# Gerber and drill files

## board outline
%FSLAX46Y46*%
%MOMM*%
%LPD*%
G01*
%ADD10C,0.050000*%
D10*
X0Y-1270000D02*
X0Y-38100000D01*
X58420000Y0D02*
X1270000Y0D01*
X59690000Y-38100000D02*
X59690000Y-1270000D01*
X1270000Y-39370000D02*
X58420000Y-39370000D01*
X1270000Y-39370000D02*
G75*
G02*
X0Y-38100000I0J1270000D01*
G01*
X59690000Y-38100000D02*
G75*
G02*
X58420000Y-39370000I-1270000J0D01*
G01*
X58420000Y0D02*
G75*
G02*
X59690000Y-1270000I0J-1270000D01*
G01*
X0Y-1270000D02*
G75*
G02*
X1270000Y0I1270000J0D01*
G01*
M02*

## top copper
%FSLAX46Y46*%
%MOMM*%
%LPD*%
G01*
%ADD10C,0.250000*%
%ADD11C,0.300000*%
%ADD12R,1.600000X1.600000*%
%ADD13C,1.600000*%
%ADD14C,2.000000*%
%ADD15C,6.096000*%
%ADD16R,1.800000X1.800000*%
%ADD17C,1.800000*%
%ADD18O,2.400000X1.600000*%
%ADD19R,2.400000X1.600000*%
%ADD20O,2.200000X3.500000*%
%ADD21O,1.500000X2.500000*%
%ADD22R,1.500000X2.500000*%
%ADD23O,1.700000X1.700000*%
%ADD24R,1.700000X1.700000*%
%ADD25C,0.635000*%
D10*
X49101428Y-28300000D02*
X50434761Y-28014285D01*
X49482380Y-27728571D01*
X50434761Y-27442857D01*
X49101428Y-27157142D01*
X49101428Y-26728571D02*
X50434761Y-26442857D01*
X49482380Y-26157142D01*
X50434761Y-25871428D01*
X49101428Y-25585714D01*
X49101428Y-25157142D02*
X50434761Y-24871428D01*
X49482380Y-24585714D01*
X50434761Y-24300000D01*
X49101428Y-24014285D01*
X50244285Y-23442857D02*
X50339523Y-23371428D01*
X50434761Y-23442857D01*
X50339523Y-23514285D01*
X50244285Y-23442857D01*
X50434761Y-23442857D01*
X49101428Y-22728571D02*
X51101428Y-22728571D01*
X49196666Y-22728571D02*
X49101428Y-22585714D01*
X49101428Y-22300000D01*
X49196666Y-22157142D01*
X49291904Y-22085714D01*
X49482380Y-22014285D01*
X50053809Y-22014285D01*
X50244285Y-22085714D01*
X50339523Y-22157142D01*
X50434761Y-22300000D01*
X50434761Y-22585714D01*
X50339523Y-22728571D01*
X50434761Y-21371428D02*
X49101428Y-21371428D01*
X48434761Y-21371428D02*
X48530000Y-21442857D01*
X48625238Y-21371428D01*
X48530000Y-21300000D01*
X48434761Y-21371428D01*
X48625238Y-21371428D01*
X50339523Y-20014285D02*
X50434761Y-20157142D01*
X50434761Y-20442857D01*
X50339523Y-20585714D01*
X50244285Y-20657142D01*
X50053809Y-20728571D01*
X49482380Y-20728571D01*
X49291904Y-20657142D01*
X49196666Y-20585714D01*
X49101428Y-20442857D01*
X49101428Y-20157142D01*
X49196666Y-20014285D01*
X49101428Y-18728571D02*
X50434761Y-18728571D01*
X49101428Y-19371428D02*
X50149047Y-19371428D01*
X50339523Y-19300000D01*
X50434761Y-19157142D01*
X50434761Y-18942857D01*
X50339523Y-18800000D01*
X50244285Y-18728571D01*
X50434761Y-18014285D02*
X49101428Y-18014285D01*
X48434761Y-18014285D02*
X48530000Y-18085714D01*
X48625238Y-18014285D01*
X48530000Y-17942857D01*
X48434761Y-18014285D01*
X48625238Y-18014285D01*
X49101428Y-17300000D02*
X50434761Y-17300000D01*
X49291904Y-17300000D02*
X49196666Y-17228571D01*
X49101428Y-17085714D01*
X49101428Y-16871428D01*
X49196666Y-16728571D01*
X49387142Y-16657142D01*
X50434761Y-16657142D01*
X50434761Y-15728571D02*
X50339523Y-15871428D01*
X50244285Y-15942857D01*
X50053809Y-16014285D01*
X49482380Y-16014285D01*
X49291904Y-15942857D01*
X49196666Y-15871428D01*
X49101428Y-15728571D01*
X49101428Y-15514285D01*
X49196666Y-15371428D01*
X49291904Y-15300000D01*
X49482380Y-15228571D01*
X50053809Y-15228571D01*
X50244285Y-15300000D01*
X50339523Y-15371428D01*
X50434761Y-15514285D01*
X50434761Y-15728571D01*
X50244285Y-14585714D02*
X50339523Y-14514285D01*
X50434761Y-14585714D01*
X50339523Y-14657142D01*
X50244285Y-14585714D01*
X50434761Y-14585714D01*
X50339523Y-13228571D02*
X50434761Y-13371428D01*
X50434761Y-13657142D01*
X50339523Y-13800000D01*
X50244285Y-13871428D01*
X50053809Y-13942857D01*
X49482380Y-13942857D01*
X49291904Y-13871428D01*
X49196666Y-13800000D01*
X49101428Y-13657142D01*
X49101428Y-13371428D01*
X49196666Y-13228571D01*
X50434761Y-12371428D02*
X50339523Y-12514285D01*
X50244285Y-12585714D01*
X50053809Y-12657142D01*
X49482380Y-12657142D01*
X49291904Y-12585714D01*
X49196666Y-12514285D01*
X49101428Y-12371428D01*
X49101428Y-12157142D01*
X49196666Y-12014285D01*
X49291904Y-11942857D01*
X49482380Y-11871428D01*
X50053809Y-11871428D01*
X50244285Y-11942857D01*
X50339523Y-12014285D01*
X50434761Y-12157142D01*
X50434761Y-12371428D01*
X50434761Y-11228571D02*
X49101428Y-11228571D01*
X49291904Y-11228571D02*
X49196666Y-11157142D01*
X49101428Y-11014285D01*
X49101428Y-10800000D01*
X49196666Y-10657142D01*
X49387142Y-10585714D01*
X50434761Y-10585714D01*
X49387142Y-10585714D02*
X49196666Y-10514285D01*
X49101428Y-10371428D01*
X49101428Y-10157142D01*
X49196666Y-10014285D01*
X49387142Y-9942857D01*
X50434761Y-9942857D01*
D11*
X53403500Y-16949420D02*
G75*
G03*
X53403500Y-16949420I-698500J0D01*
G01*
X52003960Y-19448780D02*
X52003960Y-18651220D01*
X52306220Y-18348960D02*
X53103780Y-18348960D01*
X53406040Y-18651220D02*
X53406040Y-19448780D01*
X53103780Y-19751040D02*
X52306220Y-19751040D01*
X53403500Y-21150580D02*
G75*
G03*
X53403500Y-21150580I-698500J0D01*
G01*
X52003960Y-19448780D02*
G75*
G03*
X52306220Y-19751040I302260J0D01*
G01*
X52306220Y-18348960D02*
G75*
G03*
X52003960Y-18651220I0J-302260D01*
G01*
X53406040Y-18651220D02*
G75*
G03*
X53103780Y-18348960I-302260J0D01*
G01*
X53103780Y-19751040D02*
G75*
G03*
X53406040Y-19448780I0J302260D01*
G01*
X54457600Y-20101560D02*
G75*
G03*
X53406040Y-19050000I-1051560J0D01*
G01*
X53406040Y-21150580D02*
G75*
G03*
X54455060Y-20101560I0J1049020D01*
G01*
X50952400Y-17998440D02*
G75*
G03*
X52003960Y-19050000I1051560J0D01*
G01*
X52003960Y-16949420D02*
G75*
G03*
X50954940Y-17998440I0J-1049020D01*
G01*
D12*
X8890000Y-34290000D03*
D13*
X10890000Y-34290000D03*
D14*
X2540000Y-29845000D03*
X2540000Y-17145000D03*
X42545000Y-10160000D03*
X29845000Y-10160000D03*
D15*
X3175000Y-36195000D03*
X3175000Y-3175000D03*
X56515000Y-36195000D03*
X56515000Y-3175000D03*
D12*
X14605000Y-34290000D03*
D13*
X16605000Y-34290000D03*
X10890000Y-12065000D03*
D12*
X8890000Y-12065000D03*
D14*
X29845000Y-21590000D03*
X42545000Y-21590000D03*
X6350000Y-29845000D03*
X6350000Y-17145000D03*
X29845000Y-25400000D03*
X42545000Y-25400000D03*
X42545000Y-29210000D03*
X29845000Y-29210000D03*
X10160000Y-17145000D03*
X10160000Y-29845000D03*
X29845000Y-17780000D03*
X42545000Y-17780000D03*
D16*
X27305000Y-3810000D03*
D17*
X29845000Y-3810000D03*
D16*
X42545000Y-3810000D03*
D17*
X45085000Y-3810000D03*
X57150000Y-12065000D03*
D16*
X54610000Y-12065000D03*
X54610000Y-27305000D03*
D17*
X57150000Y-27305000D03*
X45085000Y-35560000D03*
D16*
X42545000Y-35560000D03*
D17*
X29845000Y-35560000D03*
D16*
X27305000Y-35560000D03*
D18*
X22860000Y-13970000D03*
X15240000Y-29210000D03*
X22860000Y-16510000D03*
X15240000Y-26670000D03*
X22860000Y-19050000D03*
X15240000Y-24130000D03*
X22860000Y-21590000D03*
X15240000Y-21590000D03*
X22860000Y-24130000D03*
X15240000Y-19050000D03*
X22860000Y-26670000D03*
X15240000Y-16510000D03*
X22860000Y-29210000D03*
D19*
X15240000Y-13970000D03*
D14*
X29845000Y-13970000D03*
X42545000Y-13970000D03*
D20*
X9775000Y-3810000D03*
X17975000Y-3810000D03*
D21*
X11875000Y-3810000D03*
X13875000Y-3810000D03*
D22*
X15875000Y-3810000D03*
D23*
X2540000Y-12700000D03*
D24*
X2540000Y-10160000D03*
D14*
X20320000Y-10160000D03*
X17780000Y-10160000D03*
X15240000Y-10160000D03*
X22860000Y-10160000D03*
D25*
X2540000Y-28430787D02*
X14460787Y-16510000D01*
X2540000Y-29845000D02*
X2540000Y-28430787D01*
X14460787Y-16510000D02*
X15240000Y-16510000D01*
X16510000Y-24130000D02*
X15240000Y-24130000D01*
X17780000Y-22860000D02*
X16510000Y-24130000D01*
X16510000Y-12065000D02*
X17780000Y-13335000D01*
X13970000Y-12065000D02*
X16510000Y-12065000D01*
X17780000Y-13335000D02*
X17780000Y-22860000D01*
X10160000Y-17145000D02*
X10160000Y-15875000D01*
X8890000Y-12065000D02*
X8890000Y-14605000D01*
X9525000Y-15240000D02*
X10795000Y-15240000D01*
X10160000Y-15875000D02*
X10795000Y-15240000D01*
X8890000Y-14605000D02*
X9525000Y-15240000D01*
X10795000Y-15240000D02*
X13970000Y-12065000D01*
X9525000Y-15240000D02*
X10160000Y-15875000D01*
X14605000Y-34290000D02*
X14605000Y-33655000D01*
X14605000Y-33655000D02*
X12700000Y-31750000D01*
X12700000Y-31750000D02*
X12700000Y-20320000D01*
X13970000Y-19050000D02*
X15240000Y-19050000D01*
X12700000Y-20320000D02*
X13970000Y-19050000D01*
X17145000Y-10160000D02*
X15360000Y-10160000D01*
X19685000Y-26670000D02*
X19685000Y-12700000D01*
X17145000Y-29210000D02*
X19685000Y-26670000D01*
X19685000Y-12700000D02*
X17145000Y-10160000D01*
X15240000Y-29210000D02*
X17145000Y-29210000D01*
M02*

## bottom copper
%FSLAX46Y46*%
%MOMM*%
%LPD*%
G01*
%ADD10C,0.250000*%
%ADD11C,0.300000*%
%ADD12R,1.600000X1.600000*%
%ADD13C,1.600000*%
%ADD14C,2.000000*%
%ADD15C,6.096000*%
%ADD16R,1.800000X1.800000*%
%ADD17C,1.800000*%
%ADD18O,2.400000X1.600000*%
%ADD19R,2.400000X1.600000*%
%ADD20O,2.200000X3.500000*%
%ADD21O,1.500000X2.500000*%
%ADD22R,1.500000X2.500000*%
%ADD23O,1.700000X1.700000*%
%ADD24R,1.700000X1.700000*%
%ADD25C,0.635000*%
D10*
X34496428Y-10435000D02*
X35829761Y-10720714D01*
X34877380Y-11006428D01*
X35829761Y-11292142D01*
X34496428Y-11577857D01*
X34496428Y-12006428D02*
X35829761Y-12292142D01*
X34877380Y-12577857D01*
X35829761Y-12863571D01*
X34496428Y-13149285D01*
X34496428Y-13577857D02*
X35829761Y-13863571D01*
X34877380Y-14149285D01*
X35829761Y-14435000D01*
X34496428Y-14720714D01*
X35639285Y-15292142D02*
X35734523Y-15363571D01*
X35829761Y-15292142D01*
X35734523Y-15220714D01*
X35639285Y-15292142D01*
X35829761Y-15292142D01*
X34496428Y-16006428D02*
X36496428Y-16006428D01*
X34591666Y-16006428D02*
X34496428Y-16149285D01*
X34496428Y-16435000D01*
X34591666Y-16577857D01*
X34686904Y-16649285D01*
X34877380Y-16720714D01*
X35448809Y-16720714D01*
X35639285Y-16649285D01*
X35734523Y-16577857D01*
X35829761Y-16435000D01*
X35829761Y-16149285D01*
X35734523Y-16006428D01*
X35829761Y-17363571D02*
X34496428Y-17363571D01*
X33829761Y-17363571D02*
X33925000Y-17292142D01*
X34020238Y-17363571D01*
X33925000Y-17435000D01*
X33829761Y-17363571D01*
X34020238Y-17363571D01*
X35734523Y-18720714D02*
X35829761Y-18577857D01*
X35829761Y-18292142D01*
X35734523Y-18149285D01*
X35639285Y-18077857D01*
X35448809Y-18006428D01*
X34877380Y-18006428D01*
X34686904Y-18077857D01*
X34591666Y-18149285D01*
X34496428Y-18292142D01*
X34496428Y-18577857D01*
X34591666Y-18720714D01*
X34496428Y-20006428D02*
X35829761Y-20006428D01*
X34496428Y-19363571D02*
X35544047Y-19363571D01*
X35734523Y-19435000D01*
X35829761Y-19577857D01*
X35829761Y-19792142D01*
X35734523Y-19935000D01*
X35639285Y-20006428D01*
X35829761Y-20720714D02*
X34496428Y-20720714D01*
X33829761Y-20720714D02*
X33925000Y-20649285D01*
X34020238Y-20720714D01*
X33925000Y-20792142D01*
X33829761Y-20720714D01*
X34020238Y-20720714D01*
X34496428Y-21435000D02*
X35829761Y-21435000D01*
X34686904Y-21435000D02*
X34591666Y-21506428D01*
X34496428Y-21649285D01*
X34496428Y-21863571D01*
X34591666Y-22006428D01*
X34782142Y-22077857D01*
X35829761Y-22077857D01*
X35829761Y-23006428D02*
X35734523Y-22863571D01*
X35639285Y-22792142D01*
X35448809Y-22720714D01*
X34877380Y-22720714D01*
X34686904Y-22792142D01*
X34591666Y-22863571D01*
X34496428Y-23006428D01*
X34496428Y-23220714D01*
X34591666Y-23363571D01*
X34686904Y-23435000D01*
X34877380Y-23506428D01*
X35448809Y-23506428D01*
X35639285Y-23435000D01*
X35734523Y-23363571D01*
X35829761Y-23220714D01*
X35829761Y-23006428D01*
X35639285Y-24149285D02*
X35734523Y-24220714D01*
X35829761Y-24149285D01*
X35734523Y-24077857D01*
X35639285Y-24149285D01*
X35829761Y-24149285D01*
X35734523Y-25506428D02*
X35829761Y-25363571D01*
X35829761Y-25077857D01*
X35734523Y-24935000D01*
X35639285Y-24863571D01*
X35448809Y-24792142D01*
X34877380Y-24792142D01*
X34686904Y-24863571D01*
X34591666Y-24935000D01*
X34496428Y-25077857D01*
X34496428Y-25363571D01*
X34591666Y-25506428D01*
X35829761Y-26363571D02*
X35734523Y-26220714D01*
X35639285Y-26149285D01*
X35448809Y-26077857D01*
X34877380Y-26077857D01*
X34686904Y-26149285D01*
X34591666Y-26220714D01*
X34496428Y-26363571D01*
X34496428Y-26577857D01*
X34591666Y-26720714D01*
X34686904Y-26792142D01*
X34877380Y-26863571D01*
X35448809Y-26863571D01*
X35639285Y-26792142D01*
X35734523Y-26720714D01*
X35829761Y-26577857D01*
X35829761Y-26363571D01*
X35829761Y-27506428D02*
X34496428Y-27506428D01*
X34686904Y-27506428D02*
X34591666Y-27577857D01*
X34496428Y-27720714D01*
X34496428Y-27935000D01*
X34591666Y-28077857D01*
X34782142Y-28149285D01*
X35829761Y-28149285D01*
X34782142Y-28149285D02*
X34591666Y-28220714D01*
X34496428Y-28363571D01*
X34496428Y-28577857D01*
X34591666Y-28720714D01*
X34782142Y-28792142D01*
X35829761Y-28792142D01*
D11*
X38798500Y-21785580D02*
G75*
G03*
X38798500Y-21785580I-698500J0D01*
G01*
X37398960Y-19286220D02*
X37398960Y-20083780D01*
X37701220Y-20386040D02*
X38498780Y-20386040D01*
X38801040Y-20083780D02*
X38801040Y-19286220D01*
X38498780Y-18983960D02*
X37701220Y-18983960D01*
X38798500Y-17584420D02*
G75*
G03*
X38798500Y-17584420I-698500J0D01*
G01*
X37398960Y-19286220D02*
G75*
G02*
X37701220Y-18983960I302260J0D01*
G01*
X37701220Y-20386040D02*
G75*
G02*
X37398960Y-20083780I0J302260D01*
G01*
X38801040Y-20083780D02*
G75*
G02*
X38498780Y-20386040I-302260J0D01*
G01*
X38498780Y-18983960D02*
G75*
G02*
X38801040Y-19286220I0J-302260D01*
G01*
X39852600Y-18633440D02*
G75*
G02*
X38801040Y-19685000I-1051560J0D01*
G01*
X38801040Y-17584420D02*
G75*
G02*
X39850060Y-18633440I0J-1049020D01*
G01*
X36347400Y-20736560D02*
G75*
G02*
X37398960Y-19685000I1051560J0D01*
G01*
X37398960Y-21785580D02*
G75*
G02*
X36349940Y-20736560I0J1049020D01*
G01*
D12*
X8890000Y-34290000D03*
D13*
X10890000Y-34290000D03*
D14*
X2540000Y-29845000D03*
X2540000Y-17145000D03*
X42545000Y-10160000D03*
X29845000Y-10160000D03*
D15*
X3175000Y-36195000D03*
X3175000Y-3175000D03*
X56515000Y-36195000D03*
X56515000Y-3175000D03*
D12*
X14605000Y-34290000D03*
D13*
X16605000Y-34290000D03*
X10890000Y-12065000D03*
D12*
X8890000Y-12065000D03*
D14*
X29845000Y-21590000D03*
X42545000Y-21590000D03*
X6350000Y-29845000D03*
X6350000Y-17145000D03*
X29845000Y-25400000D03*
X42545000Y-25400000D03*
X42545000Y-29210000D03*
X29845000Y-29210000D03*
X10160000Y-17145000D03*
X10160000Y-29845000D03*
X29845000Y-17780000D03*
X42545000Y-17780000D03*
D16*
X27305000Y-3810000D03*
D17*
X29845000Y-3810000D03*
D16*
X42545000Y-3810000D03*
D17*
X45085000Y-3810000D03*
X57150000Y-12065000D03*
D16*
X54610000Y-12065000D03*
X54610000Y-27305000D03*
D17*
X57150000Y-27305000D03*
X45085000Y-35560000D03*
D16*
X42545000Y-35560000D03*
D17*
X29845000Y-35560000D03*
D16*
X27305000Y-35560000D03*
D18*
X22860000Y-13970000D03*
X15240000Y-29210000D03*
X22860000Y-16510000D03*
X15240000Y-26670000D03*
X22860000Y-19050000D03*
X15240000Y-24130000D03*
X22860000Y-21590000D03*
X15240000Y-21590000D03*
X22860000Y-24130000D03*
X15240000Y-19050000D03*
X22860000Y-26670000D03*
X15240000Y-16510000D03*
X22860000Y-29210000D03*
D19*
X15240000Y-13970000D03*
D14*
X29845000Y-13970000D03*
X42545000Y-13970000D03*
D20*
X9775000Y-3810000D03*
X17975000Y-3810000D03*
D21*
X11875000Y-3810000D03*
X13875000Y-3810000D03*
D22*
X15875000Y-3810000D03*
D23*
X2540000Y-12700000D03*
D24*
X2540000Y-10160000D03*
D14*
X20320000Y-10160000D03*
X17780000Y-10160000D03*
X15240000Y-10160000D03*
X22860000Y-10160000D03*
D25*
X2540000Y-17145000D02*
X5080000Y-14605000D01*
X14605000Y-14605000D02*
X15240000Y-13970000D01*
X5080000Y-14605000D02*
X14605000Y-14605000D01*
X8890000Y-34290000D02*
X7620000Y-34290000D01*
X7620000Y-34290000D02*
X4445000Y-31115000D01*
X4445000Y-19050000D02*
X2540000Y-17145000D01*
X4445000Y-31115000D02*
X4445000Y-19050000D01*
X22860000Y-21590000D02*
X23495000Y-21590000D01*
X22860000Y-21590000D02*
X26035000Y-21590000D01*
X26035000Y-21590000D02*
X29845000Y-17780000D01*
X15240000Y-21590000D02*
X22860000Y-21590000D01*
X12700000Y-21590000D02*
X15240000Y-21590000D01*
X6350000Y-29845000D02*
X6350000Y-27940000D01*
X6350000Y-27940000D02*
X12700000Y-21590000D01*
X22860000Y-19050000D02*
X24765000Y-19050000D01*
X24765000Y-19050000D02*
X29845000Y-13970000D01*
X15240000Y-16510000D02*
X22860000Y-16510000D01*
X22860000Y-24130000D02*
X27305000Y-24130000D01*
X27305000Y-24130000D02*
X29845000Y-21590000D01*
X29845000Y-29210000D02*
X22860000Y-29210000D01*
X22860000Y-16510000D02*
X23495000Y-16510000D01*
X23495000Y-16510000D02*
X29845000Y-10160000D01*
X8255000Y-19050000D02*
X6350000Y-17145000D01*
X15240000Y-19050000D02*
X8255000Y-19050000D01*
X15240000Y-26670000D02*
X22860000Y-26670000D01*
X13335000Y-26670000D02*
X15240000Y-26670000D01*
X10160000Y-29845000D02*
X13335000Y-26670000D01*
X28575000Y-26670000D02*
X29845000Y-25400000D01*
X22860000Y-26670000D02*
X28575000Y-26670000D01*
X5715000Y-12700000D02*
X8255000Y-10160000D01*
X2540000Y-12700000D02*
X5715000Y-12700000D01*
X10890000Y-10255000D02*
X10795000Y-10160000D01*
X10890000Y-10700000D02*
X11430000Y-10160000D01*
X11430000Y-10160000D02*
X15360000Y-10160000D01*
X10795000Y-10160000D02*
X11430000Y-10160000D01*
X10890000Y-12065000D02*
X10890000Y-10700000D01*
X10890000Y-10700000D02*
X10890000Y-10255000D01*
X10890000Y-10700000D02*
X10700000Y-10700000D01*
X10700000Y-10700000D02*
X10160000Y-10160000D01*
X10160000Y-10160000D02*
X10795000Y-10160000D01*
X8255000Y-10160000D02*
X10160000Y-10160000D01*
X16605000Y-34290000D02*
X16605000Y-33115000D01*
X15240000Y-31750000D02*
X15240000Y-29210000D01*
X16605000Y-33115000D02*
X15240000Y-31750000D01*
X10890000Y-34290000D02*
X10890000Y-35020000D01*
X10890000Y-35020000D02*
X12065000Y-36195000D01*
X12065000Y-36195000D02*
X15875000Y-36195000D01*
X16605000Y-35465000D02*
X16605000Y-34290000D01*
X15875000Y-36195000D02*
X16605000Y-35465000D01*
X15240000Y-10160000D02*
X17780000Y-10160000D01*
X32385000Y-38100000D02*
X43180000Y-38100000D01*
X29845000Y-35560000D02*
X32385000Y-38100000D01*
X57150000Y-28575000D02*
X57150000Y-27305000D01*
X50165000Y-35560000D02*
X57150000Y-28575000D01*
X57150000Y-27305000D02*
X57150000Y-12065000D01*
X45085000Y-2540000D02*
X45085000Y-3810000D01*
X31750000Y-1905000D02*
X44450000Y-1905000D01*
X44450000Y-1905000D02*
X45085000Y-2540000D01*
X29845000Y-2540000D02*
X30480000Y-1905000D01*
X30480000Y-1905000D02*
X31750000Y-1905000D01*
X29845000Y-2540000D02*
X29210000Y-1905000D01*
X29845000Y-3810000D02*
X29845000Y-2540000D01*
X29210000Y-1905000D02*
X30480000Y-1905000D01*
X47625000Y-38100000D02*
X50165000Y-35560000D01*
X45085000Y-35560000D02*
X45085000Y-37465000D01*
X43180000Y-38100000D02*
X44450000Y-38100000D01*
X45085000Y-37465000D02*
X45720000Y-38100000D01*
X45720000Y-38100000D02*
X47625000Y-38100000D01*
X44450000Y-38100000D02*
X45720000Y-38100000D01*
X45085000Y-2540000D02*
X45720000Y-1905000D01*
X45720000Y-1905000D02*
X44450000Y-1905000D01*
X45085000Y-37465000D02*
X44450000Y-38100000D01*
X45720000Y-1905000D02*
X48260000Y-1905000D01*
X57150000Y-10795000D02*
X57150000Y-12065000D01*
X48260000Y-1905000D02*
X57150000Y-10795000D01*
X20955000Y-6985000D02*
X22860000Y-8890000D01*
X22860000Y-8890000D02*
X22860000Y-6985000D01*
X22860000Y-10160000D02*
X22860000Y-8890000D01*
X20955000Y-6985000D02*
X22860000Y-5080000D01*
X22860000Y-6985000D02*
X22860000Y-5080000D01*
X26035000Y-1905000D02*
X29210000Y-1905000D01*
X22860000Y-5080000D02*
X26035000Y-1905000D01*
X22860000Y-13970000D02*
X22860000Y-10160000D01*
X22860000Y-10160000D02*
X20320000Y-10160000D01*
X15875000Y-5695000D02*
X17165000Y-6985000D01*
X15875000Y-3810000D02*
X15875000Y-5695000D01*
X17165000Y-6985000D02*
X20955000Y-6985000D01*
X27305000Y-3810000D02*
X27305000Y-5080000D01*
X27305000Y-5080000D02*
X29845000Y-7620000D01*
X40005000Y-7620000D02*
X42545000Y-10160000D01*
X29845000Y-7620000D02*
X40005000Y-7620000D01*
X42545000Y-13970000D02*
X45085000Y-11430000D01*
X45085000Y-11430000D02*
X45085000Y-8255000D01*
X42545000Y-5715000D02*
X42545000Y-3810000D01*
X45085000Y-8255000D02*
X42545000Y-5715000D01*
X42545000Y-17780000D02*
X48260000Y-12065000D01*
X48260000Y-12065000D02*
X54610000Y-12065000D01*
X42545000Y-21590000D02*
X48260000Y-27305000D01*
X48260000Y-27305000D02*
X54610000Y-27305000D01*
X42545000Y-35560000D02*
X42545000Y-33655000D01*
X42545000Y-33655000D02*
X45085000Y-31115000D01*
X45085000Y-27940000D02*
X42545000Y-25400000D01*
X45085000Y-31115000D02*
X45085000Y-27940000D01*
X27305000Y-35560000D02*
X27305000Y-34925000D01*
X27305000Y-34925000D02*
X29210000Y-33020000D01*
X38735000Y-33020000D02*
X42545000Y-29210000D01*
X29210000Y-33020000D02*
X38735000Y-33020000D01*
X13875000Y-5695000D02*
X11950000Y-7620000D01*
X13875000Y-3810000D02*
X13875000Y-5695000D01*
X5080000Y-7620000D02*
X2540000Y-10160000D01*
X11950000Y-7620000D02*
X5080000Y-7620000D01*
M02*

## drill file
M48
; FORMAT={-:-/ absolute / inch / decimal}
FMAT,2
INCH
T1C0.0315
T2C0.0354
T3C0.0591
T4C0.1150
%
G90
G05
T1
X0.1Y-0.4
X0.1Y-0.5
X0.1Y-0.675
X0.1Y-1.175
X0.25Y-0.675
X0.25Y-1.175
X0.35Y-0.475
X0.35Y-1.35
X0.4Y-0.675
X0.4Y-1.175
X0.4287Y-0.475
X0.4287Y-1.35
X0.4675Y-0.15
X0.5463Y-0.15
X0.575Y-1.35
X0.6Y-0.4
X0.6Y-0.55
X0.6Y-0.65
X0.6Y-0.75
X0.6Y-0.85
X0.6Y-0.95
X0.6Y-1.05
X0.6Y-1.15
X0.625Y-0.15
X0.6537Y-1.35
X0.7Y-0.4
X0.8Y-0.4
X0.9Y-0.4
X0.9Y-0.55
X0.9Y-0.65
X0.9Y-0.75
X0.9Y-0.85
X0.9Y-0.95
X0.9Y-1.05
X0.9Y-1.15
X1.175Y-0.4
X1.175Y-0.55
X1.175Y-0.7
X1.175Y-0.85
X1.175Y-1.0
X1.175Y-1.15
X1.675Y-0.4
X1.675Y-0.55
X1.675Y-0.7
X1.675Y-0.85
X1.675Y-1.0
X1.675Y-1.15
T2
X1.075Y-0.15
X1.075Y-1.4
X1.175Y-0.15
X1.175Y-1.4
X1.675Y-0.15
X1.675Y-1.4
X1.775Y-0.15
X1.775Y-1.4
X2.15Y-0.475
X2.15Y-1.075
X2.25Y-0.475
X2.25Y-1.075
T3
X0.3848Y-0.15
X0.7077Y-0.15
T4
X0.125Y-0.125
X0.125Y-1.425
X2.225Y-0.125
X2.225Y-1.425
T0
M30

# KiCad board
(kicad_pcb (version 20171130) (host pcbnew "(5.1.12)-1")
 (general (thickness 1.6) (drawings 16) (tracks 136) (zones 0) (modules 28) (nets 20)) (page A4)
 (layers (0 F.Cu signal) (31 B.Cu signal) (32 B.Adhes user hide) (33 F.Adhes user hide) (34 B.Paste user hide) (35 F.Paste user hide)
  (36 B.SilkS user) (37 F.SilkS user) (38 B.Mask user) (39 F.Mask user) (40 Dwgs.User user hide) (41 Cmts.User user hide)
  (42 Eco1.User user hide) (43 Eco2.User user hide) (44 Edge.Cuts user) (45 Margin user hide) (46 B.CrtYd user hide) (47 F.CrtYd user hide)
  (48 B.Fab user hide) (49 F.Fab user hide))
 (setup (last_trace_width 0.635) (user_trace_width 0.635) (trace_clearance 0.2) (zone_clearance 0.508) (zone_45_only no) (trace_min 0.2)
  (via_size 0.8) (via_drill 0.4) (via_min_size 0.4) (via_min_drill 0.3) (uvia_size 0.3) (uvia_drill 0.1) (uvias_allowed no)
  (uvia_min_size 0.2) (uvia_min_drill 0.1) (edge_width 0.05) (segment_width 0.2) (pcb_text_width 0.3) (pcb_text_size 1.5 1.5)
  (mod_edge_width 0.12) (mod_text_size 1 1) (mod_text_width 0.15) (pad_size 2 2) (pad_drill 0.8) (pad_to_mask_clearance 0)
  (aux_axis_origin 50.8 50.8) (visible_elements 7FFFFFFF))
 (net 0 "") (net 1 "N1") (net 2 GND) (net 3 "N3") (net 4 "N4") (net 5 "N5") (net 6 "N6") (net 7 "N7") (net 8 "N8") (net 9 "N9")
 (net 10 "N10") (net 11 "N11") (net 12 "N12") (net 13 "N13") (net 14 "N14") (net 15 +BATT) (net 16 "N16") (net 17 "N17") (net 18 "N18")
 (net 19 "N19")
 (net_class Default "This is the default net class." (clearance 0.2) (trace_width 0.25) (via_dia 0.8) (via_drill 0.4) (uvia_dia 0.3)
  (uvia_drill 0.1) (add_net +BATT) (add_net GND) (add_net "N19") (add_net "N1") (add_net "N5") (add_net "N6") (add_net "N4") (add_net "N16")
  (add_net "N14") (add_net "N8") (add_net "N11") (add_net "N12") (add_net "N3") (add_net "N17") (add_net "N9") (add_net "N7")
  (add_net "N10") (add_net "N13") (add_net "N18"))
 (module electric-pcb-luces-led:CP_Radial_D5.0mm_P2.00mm (layer F.Cu) (at 59.69 85.09)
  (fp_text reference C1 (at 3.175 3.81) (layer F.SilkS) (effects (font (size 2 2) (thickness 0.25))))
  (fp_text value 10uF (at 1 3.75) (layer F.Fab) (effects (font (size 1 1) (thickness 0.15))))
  (pad 1 thru_hole rect (at 0 0) (size 1.6 1.6) (drill 0.8) (layers *.Cu *.Mask) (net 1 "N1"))
  (pad 2 thru_hole circle (at 2 0) (size 1.6 1.6) (drill 0.8) (layers *.Cu *.Mask) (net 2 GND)))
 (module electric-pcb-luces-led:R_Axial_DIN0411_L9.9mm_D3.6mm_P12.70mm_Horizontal (layer F.Cu) (at 53.34 80.645 90)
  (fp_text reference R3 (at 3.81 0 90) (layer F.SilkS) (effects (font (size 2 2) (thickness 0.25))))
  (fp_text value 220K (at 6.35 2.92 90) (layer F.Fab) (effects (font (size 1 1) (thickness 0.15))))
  (pad 1 thru_hole circle (at 0 0 90) (size 2 2) (drill 0.8) (layers *.Cu *.Mask) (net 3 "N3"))
  (pad 2 thru_hole circle (at 12.7 0 90) (size 2 2) (drill 0.8) (layers *.Cu *.Mask) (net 1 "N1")))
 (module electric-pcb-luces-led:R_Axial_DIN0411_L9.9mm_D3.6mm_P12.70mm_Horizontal (layer F.Cu) (at 93.345 60.96 180)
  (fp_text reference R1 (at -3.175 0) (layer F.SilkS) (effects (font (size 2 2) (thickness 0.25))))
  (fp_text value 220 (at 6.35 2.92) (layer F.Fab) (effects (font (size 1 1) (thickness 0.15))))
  (pad 1 thru_hole circle (at 0 0 180) (size 2 2) (drill 0.8) (layers *.Cu *.Mask) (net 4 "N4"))
  (pad 2 thru_hole circle (at 12.7 0 180) (size 2 2) (drill 0.8) (layers *.Cu *.Mask) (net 3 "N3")))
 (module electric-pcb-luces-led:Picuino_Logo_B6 (layer B.Cu) (at 103.505 69.85 270)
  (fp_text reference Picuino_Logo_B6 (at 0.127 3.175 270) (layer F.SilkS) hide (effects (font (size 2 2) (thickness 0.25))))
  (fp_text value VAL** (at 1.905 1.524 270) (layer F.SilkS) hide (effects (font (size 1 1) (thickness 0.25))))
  (fp_circle (center -2.10058 0) (end -1.40208 0) (layer F.Cu) (width 0.3))
  (fp_line (start 0.39878 0.70104) (end -0.39878 0.70104) (layer F.Cu) (width 0.3))
  (fp_line (start -0.70104 0.39878) (end -0.70104 -0.39878) (layer F.Cu) (width 0.3))
  (fp_line (start -0.39878 -0.70104) (end 0.39878 -0.70104) (layer F.Cu) (width 0.3))
  (fp_line (start 0.70104 -0.39878) (end 0.70104 0.39878) (layer F.Cu) (width 0.3))
  (fp_circle (center 2.10058 0) (end 2.79908 0) (layer F.Cu) (width 0.3))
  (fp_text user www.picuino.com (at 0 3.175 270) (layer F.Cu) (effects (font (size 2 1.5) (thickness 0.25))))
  (fp_arc (start 0.39878 0.39878) (end 0.70104 0.39878) (angle 90) (layer F.Cu) (width 0.3))
  (fp_arc (start -0.39878 0.39878) (end -0.39878 0.70104) (angle 90) (layer F.Cu) (width 0.3))
  (fp_arc (start -0.39878 -0.39878) (end -0.70104 -0.39878) (angle 90) (layer F.Cu) (width 0.3))
  (fp_arc (start 0.39878 -0.39878) (end 0.39878 -0.70104) (angle 90) (layer F.Cu) (width 0.3))
  (fp_arc (start 1.05156 -0.70104) (end 0 -0.70104) (angle 90) (layer F.Cu) (width 0.3))
  (fp_arc (start 1.05156 -0.70104) (end 1.05156 -1.75006) (angle 90) (layer F.Cu) (width 0.3))
  (fp_arc (start -1.05156 0.70104) (end 0 0.70104) (angle 90) (layer F.Cu) (width 0.3))
  (fp_arc (start -1.05156 0.70104) (end -1.05156 1.75006) (angle 90) (layer F.Cu) (width 0.3)))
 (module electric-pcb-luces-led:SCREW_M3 (layer F.Cu) (at 53.975 86.995)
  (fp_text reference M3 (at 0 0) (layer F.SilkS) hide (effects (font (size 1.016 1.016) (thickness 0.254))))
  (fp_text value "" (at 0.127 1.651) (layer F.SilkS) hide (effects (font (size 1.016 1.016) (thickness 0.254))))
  (pad "" thru_hole circle (at 0 0) (size 6.096 6.096) (drill 2.921) (layers *.Cu F.SilkS)))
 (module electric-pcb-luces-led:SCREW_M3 (layer F.Cu) (at 53.975 53.975)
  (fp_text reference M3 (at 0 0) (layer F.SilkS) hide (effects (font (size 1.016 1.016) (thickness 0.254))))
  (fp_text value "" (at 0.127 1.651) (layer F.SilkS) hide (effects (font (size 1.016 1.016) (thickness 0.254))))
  (pad "" thru_hole circle (at 0 0) (size 6.096 6.096) (drill 2.921) (layers *.Cu F.SilkS)))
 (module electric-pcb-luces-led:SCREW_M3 (layer F.Cu) (at 107.315 86.995)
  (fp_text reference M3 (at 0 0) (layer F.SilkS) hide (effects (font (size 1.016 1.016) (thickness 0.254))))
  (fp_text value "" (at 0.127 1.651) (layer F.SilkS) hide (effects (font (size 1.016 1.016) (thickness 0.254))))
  (pad "" thru_hole circle (at 0 0) (size 6.096 6.096) (drill 2.921) (layers *.Cu F.SilkS)))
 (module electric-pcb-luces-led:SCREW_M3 (layer F.Cu) (at 107.315 53.975)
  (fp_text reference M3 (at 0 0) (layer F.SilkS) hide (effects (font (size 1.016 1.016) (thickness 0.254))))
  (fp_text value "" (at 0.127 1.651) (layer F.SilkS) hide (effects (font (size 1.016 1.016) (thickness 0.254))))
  (pad "" thru_hole circle (at 0 0) (size 6.096 6.096) (drill 2.921) (layers *.Cu F.SilkS)))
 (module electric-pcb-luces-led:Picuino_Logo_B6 (layer F.Cu) (at 88.9 70.485 90)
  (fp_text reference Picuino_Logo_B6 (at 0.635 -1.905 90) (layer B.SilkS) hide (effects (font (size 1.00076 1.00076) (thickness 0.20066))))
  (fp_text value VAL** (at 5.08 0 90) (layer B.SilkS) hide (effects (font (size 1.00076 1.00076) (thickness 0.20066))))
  (fp_circle (center -2.10058 0) (end -1.40208 0) (layer B.Cu) (width 0.3))
  (fp_line (start 0.39878 -0.70104) (end -0.39878 -0.70104) (layer B.Cu) (width 0.3))
  (fp_line (start -0.70104 -0.39878) (end -0.70104 0.39878) (layer B.Cu) (width 0.3))
  (fp_line (start -0.39878 0.70104) (end 0.39878 0.70104) (layer B.Cu) (width 0.3))
  (fp_line (start 0.70104 0.39878) (end 0.70104 -0.39878) (layer B.Cu) (width 0.3))
  (fp_circle (center 2.10058 0) (end 2.79908 0) (layer B.Cu) (width 0.3))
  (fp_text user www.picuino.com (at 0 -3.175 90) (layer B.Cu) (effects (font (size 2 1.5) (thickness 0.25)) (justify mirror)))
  (fp_arc (start 0.39878 -0.39878) (end 0.70104 -0.39878) (angle -90) (layer B.Cu) (width 0.3))
  (fp_arc (start -0.39878 -0.39878) (end -0.39878 -0.70104) (angle -90) (layer B.Cu) (width 0.3))
  (fp_arc (start -0.39878 0.39878) (end -0.70104 0.39878) (angle -90) (layer B.Cu) (width 0.3))
  (fp_arc (start 0.39878 0.39878) (end 0.39878 0.70104) (angle -90) (layer B.Cu) (width 0.3))
  (fp_arc (start 1.05156 0.70104) (end 0 0.70104) (angle -90) (layer B.Cu) (width 0.3))
  (fp_arc (start 1.05156 0.70104) (end 1.05156 1.75006) (angle -90) (layer B.Cu) (width 0.3))
  (fp_arc (start -1.05156 -0.70104) (end 0 -0.70104) (angle -90) (layer B.Cu) (width 0.3))
  (fp_arc (start -1.05156 -0.70104) (end -1.05156 -1.75006) (angle -90) (layer B.Cu) (width 0.3)))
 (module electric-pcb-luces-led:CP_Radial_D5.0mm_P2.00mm (layer F.Cu) (at 65.405 85.09)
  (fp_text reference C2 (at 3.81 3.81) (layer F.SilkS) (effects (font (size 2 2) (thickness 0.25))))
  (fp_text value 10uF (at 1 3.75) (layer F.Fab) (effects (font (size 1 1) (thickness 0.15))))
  (pad 1 thru_hole rect (at 0 0) (size 1.6 1.6) (drill 0.8) (layers *.Cu *.Mask) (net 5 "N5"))
  (pad 2 thru_hole circle (at 2 0) (size 1.6 1.6) (drill 0.8) (layers *.Cu *.Mask) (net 2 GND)))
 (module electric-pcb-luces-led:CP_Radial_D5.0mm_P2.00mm (layer F.Cu) (at 59.69 62.865)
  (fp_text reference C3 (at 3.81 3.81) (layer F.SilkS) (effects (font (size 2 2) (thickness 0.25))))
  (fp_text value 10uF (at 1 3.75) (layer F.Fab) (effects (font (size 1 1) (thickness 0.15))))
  (pad 2 thru_hole circle (at 2 0) (size 1.6 1.6) (drill 0.8) (layers *.Cu *.Mask) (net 2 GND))
  (pad 1 thru_hole rect (at 0 0) (size 1.6 1.6) (drill 0.8) (layers *.Cu *.Mask) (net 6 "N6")))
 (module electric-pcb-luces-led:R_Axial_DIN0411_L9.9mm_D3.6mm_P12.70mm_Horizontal (layer F.Cu) (at 93.345 72.39 180)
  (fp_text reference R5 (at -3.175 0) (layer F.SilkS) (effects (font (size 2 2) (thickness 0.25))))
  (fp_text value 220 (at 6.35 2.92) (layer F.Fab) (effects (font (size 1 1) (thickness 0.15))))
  (pad 2 thru_hole circle (at 12.7 0 180) (size 2 2) (drill 0.8) (layers *.Cu *.Mask) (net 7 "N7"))
  (pad 1 thru_hole circle (at 0 0 180) (size 2 2) (drill 0.8) (layers *.Cu *.Mask) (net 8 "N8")))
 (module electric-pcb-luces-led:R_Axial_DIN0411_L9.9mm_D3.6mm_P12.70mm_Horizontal (layer F.Cu) (at 57.15 80.645 90)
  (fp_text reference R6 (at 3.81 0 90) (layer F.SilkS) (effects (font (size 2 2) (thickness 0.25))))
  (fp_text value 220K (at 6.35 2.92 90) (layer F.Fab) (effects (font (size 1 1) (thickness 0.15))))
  (pad 1 thru_hole circle (at 0 0 90) (size 2 2) (drill 0.8) (layers *.Cu *.Mask) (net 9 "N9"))
  (pad 2 thru_hole circle (at 12.7 0 90) (size 2 2) (drill 0.8) (layers *.Cu *.Mask) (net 5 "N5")))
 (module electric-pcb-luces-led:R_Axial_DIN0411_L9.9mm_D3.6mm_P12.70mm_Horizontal (layer F.Cu) (at 93.345 76.2 180)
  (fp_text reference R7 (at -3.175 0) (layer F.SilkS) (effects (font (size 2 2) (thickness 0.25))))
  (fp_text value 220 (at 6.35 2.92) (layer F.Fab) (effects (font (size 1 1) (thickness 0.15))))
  (pad 2 thru_hole circle (at 12.7 0 180) (size 2 2) (drill 0.8) (layers *.Cu *.Mask) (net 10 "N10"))
  (pad 1 thru_hole circle (at 0 0 180) (size 2 2) (drill 0.8) (layers *.Cu *.Mask) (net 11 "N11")))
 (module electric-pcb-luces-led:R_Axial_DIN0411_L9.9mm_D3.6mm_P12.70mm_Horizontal (layer F.Cu) (at 93.345 80.01 180)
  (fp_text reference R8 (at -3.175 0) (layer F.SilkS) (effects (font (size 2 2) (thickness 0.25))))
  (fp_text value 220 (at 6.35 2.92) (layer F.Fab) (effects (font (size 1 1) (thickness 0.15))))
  (pad 1 thru_hole circle (at 0 0 180) (size 2 2) (drill 0.8) (layers *.Cu *.Mask) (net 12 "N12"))
  (pad 2 thru_hole circle (at 12.7 0 180) (size 2 2) (drill 0.8) (layers *.Cu *.Mask) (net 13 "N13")))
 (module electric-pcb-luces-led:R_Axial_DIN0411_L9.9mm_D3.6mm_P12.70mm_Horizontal (layer F.Cu) (at 60.96 80.645 90)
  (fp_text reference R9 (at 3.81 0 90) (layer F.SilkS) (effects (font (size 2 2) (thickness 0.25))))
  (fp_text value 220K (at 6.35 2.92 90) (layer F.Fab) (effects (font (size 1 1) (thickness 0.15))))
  (pad 2 thru_hole circle (at 12.7 0 90) (size 2 2) (drill 0.8) (layers *.Cu *.Mask) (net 6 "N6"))
  (pad 1 thru_hole circle (at 0 0 90) (size 2 2) (drill 0.8) (layers *.Cu *.Mask) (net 10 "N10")))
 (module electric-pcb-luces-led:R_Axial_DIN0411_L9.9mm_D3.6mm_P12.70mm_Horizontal (layer F.Cu) (at 93.345 68.58 180)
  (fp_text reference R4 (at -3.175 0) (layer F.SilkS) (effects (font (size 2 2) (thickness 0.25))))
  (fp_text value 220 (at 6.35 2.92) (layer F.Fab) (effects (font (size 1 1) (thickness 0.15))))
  (pad 2 thru_hole circle (at 12.7 0 180) (size 2 2) (drill 0.8) (layers *.Cu *.Mask) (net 9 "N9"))
  (pad 1 thru_hole circle (at 0 0 180) (size 2 2) (drill 0.8) (layers *.Cu *.Mask) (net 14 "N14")))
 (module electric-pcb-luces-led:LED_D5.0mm (layer F.Cu) (at 78.105 54.61)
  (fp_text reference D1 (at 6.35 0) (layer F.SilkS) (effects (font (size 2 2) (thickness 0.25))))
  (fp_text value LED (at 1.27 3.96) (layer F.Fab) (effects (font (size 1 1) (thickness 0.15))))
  (pad 1 thru_hole rect (at 0 0) (size 1.8 1.8) (drill 0.9) (layers *.Cu *.Mask) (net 4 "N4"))
  (pad 2 thru_hole circle (at 2.54 0) (size 1.8 1.8) (drill 0.9) (layers *.Cu *.Mask) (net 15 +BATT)))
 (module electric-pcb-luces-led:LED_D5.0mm (layer F.Cu) (at 93.345 54.61)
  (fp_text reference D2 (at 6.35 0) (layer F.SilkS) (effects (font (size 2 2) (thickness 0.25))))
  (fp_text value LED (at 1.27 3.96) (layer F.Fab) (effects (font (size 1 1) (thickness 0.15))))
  (pad 1 thru_hole rect (at 0 0) (size 1.8 1.8) (drill 0.9) (layers *.Cu *.Mask) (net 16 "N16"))
  (pad 2 thru_hole circle (at 2.54 0) (size 1.8 1.8) (drill 0.9) (layers *.Cu *.Mask) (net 15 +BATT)))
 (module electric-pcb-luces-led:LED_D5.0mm (layer F.Cu) (at 105.41 62.865)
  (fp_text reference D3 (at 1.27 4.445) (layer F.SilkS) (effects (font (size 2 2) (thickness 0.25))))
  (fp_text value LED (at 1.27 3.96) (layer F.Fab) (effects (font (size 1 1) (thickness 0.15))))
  (pad 2 thru_hole circle (at 2.54 0) (size 1.8 1.8) (drill 0.9) (layers *.Cu *.Mask) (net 15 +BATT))
  (pad 1 thru_hole rect (at 0 0) (size 1.8 1.8) (drill 0.9) (layers *.Cu *.Mask) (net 14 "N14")))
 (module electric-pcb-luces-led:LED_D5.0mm (layer F.Cu) (at 105.41 78.105)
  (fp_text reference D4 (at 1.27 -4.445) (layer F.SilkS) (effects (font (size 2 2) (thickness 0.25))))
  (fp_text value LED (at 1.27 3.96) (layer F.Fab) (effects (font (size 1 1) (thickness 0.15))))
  (pad 1 thru_hole rect (at 0 0) (size 1.8 1.8) (drill 0.9) (layers *.Cu *.Mask) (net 8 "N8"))
  (pad 2 thru_hole circle (at 2.54 0) (size 1.8 1.8) (drill 0.9) (layers *.Cu *.Mask) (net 15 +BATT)))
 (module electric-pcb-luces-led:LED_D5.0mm (layer F.Cu) (at 93.345 86.36)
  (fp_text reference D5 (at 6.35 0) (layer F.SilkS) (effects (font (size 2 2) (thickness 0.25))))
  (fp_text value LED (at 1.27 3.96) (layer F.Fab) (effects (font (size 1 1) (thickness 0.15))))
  (pad 2 thru_hole circle (at 2.54 0) (size 1.8 1.8) (drill 0.9) (layers *.Cu *.Mask) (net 15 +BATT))
  (pad 1 thru_hole rect (at 0 0) (size 1.8 1.8) (drill 0.9) (layers *.Cu *.Mask) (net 11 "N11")))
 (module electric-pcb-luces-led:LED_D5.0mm (layer F.Cu) (at 78.105 86.36)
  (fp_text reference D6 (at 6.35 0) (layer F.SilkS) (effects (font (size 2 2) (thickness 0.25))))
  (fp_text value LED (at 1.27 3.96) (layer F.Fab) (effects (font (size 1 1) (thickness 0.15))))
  (pad 2 thru_hole circle (at 2.54 0) (size 1.8 1.8) (drill 0.9) (layers *.Cu *.Mask) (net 15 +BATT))
  (pad 1 thru_hole rect (at 0 0) (size 1.8 1.8) (drill 0.9) (layers *.Cu *.Mask) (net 12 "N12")))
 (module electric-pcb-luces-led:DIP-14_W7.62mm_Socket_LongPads (layer F.Cu) (at 66.04 64.77)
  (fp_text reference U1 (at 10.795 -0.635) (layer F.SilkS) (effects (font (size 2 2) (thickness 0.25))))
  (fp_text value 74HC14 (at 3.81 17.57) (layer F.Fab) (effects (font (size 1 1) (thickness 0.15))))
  (pad 14 thru_hole oval (at 7.62 0) (size 2.4 1.6) (drill 0.8) (layers *.Cu *.Mask) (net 15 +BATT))
  (pad 7 thru_hole oval (at 0 15.24) (size 2.4 1.6) (drill 0.8) (layers *.Cu *.Mask) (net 2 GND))
  (pad 13 thru_hole oval (at 7.62 2.54) (size 2.4 1.6) (drill 0.8) (layers *.Cu *.Mask) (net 3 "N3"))
  (pad 6 thru_hole oval (at 0 12.7) (size 2.4 1.6) (drill 0.8) (layers *.Cu *.Mask) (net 10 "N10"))
  (pad 12 thru_hole oval (at 7.62 5.08) (size 2.4 1.6) (drill 0.8) (layers *.Cu *.Mask) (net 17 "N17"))
  (pad 5 thru_hole oval (at 0 10.16) (size 2.4 1.6) (drill 0.8) (layers *.Cu *.Mask) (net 6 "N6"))
  (pad 11 thru_hole oval (at 7.62 7.62) (size 2.4 1.6) (drill 0.8) (layers *.Cu *.Mask) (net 9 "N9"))
  (pad 4 thru_hole oval (at 0 7.62) (size 2.4 1.6) (drill 0.8) (layers *.Cu *.Mask) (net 9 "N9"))
  (pad 10 thru_hole oval (at 7.62 10.16) (size 2.4 1.6) (drill 0.8) (layers *.Cu *.Mask) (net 7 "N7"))
  (pad 3 thru_hole oval (at 0 5.08) (size 2.4 1.6) (drill 0.8) (layers *.Cu *.Mask) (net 5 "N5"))
  (pad 9 thru_hole oval (at 7.62 12.7) (size 2.4 1.6) (drill 0.8) (layers *.Cu *.Mask) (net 10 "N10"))
  (pad 2 thru_hole oval (at 0 2.54) (size 2.4 1.6) (drill 0.8) (layers *.Cu *.Mask) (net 3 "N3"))
  (pad 8 thru_hole oval (at 7.62 15.24) (size 2.4 1.6) (drill 0.8) (layers *.Cu *.Mask) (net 13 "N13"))
  (pad 1 thru_hole rect (at 0 0) (size 2.4 1.6) (drill 0.8) (layers *.Cu *.Mask) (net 1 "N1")))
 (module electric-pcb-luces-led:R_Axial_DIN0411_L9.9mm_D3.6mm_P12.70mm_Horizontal (layer F.Cu) (at 93.345 64.77 180)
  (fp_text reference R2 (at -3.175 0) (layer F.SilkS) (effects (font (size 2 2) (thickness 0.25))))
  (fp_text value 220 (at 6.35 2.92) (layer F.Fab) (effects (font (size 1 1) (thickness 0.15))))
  (pad 2 thru_hole circle (at 12.7 0 180) (size 2 2) (drill 0.8) (layers *.Cu *.Mask) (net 17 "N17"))
  (pad 1 thru_hole circle (at 0 0 180) (size 2 2) (drill 0.8) (layers *.Cu *.Mask) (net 16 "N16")))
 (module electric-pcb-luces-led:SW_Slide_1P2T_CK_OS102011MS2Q (layer F.Cu) (at 66.675 54.61 180)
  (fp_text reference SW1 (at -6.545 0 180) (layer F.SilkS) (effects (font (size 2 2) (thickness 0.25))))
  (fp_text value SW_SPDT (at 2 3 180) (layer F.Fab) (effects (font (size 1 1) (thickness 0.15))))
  (pad "" thru_hole oval (at 6.1 0 180) (size 2.2 3.5) (drill 1.5) (layers *.Cu *.Mask))
  (pad "" thru_hole oval (at -2.1 0 180) (size 2.2 3.5) (drill 1.5) (layers *.Cu *.Mask))
  (pad 3 thru_hole oval (at 4 0 180) (size 1.5 2.5) (drill 0.8) (layers *.Cu *.Mask) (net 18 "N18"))
  (pad 2 thru_hole oval (at 2 0 180) (size 1.5 2.5) (drill 0.8) (layers *.Cu *.Mask) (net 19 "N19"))
  (pad 1 thru_hole rect (at 0 0 180) (size 1.5 2.5) (drill 0.8) (layers *.Cu *.Mask) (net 15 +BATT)))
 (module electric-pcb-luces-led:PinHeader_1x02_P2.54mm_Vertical (layer F.Cu) (at 53.34 60.96)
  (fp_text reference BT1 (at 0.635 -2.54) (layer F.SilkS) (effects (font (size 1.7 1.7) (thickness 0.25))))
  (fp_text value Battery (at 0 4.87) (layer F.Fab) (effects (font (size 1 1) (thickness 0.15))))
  (pad 2 thru_hole oval (at 0 2.54) (size 1.7 1.7) (drill 0.8) (layers *.Cu *.Mask) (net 2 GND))
  (pad 1 thru_hole rect (at 0 0) (size 1.7 1.7) (drill 0.8) (layers *.Cu *.Mask) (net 19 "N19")))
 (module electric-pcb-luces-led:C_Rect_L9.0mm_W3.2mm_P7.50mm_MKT (layer F.Cu) (at 73.66 60.96 180)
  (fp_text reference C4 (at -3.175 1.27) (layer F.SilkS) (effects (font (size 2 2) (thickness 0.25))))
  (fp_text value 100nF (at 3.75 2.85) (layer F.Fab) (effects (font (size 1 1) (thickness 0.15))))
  (pad 1 thru_hole circle (at 2.54 0 180) (size 2 2) (drill 0.8) (layers *.Cu *.Mask) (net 15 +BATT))
  (pad 2 thru_hole circle (at 5.08 0 180) (size 2 2) (drill 0.8) (layers *.Cu *.Mask) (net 2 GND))
  (pad 2 thru_hole circle (at 7.62 0 180) (size 2 2) (drill 0.8) (layers *.Cu *.Mask) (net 2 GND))
  (pad 1 thru_hole circle (at 0 0 180) (size 2 2) (drill 0.8) (layers *.Cu *.Mask) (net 15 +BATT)))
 (gr_line (start 50.8 52.07) (end 50.8 88.9) (layer Edge.Cuts) (width 0.05))
 (gr_line (start 109.22 50.8) (end 52.07 50.8) (layer Edge.Cuts) (width 0.05))
 (gr_line (start 110.49 88.9) (end 110.49 52.07) (layer Edge.Cuts) (width 0.05))
 (gr_line (start 52.07 90.17) (end 109.22 90.17) (layer Edge.Cuts) (width 0.05))
 (gr_arc (start 52.07 88.9) (end 50.8 88.9) (angle -90) (layer Edge.Cuts) (width 0.05))
 (gr_arc (start 109.22 88.9) (end 109.22 90.17) (angle -90) (layer Edge.Cuts) (width 0.05))
 (gr_arc (start 109.22 52.07) (end 110.49 52.07) (angle -90) (layer Edge.Cuts) (width 0.05))
 (gr_arc (start 52.07 52.07) (end 52.07 50.8) (angle -90) (layer Edge.Cuts) (width 0.05))
 (segment (start 53.34 67.945) (end 55.88 65.405) (width 0.635) (layer B.Cu) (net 1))
 (segment (start 65.405 65.405) (end 66.04 64.77) (width 0.635) (layer B.Cu) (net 1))
 (segment (start 55.88 65.405) (end 65.405 65.405) (width 0.635) (layer B.Cu) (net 1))
 (segment (start 59.69 85.09) (end 58.42 85.09) (width 0.635) (layer B.Cu) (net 1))
 (segment (start 58.42 85.09) (end 55.245 81.915) (width 0.635) (layer B.Cu) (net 1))
 (segment (start 55.245 69.85) (end 53.34 67.945) (width 0.635) (layer B.Cu) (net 1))
 (segment (start 55.245 81.915) (end 55.245 69.85) (width 0.635) (layer B.Cu) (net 1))
 (segment (start 73.66 72.39) (end 74.295 72.39) (width 0.635) (layer B.Cu) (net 9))
 (segment (start 73.66 72.39) (end 76.835 72.39) (width 0.635) (layer B.Cu) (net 9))
 (segment (start 76.835 72.39) (end 80.645 68.58) (width 0.635) (layer B.Cu) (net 9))
 (segment (start 66.04 72.39) (end 73.66 72.39) (width 0.635) (layer B.Cu) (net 9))
 (segment (start 63.5 72.39) (end 66.04 72.39) (width 0.635) (layer B.Cu) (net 9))
 (segment (start 57.15 80.645) (end 57.15 78.74) (width 0.635) (layer B.Cu) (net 9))
 (segment (start 57.15 78.74) (end 63.5 72.39) (width 0.635) (layer B.Cu) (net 9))
 (segment (start 73.66 69.85) (end 75.565 69.85) (width 0.635) (layer B.Cu) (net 17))
 (segment (start 75.565 69.85) (end 80.645 64.77) (width 0.635) (layer B.Cu) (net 17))
 (segment (start 66.04 67.31) (end 73.66 67.31) (width 0.635) (layer B.Cu) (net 3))
 (segment (start 73.66 74.93) (end 78.105 74.93) (width 0.635) (layer B.Cu) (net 7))
 (segment (start 78.105 74.93) (end 80.645 72.39) (width 0.635) (layer B.Cu) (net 7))
 (segment (start 80.645 80.01) (end 73.66 80.01) (width 0.635) (layer B.Cu) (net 13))
 (segment (start 53.34 79.230787) (end 65.260787 67.31) (width 0.635) (layer F.Cu) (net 3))
 (segment (start 53.34 80.645) (end 53.34 79.230787) (width 0.635) (layer F.Cu) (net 3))
 (segment (start 65.260787 67.31) (end 66.04 67.31) (width 0.635) (layer F.Cu) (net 3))
 (segment (start 73.66 67.31) (end 74.295 67.31) (width 0.635) (layer B.Cu) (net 3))
 (segment (start 74.295 67.31) (end 80.645 60.96) (width 0.635) (layer B.Cu) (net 3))
 (segment (start 67.31 74.93) (end 66.04 74.93) (width 0.635) (layer F.Cu) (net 6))
 (segment (start 68.58 73.66) (end 67.31 74.93) (width 0.635) (layer F.Cu) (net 6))
 (segment (start 67.31 62.865) (end 68.58 64.135) (width 0.635) (layer F.Cu) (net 6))
 (segment (start 64.77 62.865) (end 67.31 62.865) (width 0.635) (layer F.Cu) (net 6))
 (segment (start 68.58 64.135) (end 68.58 73.66) (width 0.635) (layer F.Cu) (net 6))
 (segment (start 60.96 67.945) (end 60.96 66.675) (width 0.635) (layer F.Cu) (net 6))
 (segment (start 59.69 62.865) (end 59.69 65.405) (width 0.635) (layer F.Cu) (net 6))
 (segment (start 60.325 66.04) (end 61.595 66.04) (width 0.635) (layer F.Cu) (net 6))
 (segment (start 60.96 66.675) (end 61.595 66.04) (width 0.635) (layer F.Cu) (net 6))
 (segment (start 59.69 65.405) (end 60.325 66.04) (width 0.635) (layer F.Cu) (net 6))
 (segment (start 61.595 66.04) (end 64.77 62.865) (width 0.635) (layer F.Cu) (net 6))
 (segment (start 60.325 66.04) (end 60.96 66.675) (width 0.635) (layer F.Cu) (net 6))
 (segment (start 59.055 69.85) (end 57.15 67.945) (width 0.635) (layer B.Cu) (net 5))
 (segment (start 66.04 69.85) (end 59.055 69.85) (width 0.635) (layer B.Cu) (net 5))
 (segment (start 65.405 85.09) (end 65.405 84.455) (width 0.635) (layer F.Cu) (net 5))
 (segment (start 65.405 84.455) (end 63.5 82.55) (width 0.635) (layer F.Cu) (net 5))
 (segment (start 63.5 82.55) (end 63.5 71.12) (width 0.635) (layer F.Cu) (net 5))
 (segment (start 64.77 69.85) (end 66.04 69.85) (width 0.635) (layer F.Cu) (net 5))
 (segment (start 63.5 71.12) (end 64.77 69.85) (width 0.635) (layer F.Cu) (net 5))
 (segment (start 66.04 77.47) (end 73.66 77.47) (width 0.635) (layer B.Cu) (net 10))
 (segment (start 64.135 77.47) (end 66.04 77.47) (width 0.635) (layer B.Cu) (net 10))
 (segment (start 60.96 80.645) (end 64.135 77.47) (width 0.635) (layer B.Cu) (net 10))
 (segment (start 79.375 77.47) (end 80.645 76.2) (width 0.635) (layer B.Cu) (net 10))
 (segment (start 73.66 77.47) (end 79.375 77.47) (width 0.635) (layer B.Cu) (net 10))
 (segment (start 67.945 60.96) (end 66.16 60.96) (width 0.635) (layer F.Cu) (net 2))
 (segment (start 70.485 77.47) (end 70.485 63.5) (width 0.635) (layer F.Cu) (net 2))
 (segment (start 67.945 80.01) (end 70.485 77.47) (width 0.635) (layer F.Cu) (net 2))
 (segment (start 70.485 63.5) (end 67.945 60.96) (width 0.635) (layer F.Cu) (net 2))
 (segment (start 66.04 80.01) (end 67.945 80.01) (width 0.635) (layer F.Cu) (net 2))
 (segment (start 56.515 63.5) (end 59.055 60.96) (width 0.635) (layer B.Cu) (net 2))
 (segment (start 53.34 63.5) (end 56.515 63.5) (width 0.635) (layer B.Cu) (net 2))
 (segment (start 61.69 61.055) (end 61.595 60.96) (width 0.635) (layer B.Cu) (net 2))
 (segment (start 61.69 61.5) (end 62.23 60.96) (width 0.635) (layer B.Cu) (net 2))
 (segment (start 62.23 60.96) (end 66.16 60.96) (width 0.635) (layer B.Cu) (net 2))
 (segment (start 61.595 60.96) (end 62.23 60.96) (width 0.635) (layer B.Cu) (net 2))
 (segment (start 61.69 62.865) (end 61.69 61.5) (width 0.635) (layer B.Cu) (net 2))
 (segment (start 61.69 61.5) (end 61.69 61.055) (width 0.635) (layer B.Cu) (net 2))
 (segment (start 61.69 61.5) (end 61.5 61.5) (width 0.635) (layer B.Cu) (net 2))
 (segment (start 61.5 61.5) (end 60.96 60.96) (width 0.635) (layer B.Cu) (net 2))
 (segment (start 60.96 60.96) (end 61.595 60.96) (width 0.635) (layer B.Cu) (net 2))
 (segment (start 59.055 60.96) (end 60.96 60.96) (width 0.635) (layer B.Cu) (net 2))
 (segment (start 67.405 85.09) (end 67.405 83.915) (width 0.635) (layer B.Cu) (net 2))
 (segment (start 66.04 82.55) (end 66.04 80.01) (width 0.635) (layer B.Cu) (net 2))
 (segment (start 67.405 83.915) (end 66.04 82.55) (width 0.635) (layer B.Cu) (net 2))
 (segment (start 61.69 85.09) (end 61.69 85.82) (width 0.635) (layer B.Cu) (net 2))
 (segment (start 61.69 85.82) (end 62.865 86.995) (width 0.635) (layer B.Cu) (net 2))
 (segment (start 62.865 86.995) (end 66.675 86.995) (width 0.635) (layer B.Cu) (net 2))
 (segment (start 67.405 86.265) (end 67.405 85.09) (width 0.635) (layer B.Cu) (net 2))
 (segment (start 66.675 86.995) (end 67.405 86.265) (width 0.635) (layer B.Cu) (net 2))
 (segment (start 66.04 60.96) (end 68.58 60.96) (width 0.635) (layer B.Cu) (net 2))
 (segment (start 83.185 88.9) (end 93.98 88.9) (width 0.635) (layer B.Cu) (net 15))
 (segment (start 80.645 86.36) (end 83.185 88.9) (width 0.635) (layer B.Cu) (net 15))
 (segment (start 107.95 79.375) (end 107.95 78.105) (width 0.635) (layer B.Cu) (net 15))
 (segment (start 100.965 86.36) (end 107.95 79.375) (width 0.635) (layer B.Cu) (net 15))
 (segment (start 107.95 78.105) (end 107.95 62.865) (width 0.635) (layer B.Cu) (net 15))
 (segment (start 95.885 53.34) (end 95.885 54.61) (width 0.635) (layer B.Cu) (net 15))
 (segment (start 82.55 52.705) (end 95.25 52.705) (width 0.635) (layer B.Cu) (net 15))
 (segment (start 95.25 52.705) (end 95.885 53.34) (width 0.635) (layer B.Cu) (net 15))
 (segment (start 80.645 53.34) (end 81.28 52.705) (width 0.635) (layer B.Cu) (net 15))
 (segment (start 81.28 52.705) (end 82.55 52.705) (width 0.635) (layer B.Cu) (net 15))
 (segment (start 80.645 53.34) (end 80.01 52.705) (width 0.635) (layer B.Cu) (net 15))
 (segment (start 80.645 54.61) (end 80.645 53.34) (width 0.635) (layer B.Cu) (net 15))
 (segment (start 80.01 52.705) (end 81.28 52.705) (width 0.635) (layer B.Cu) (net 15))
 (segment (start 98.425 88.9) (end 100.965 86.36) (width 0.635) (layer B.Cu) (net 15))
 (segment (start 95.885 86.36) (end 95.885 88.265) (width 0.635) (layer B.Cu) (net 15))
 (segment (start 93.98 88.9) (end 95.25 88.9) (width 0.635) (layer B.Cu) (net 15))
 (segment (start 95.885 88.265) (end 96.52 88.9) (width 0.635) (layer B.Cu) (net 15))
 (segment (start 96.52 88.9) (end 98.425 88.9) (width 0.635) (layer B.Cu) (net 15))
 (segment (start 95.25 88.9) (end 96.52 88.9) (width 0.635) (layer B.Cu) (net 15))
 (segment (start 95.885 53.34) (end 96.52 52.705) (width 0.635) (layer B.Cu) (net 15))
 (segment (start 96.52 52.705) (end 95.25 52.705) (width 0.635) (layer B.Cu) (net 15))
 (segment (start 95.885 88.265) (end 95.25 88.9) (width 0.635) (layer B.Cu) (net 15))
 (segment (start 96.52 52.705) (end 99.06 52.705) (width 0.635) (layer B.Cu) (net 15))
 (segment (start 107.95 61.595) (end 107.95 62.865) (width 0.635) (layer B.Cu) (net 15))
 (segment (start 99.06 52.705) (end 107.95 61.595) (width 0.635) (layer B.Cu) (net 15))
 (segment (start 71.755 57.785) (end 73.66 59.69) (width 0.635) (layer B.Cu) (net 15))
 (segment (start 73.66 59.69) (end 73.66 57.785) (width 0.635) (layer B.Cu) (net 15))
 (segment (start 73.66 60.96) (end 73.66 59.69) (width 0.635) (layer B.Cu) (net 15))
 (segment (start 71.755 57.785) (end 73.66 55.88) (width 0.635) (layer B.Cu) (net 15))
 (segment (start 73.66 57.785) (end 73.66 55.88) (width 0.635) (layer B.Cu) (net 15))
 (segment (start 76.835 52.705) (end 80.01 52.705) (width 0.635) (layer B.Cu) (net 15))
 (segment (start 73.66 55.88) (end 76.835 52.705) (width 0.635) (layer B.Cu) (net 15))
 (segment (start 73.66 64.77) (end 73.66 60.96) (width 0.635) (layer B.Cu) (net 15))
 (segment (start 73.66 60.96) (end 71.12 60.96) (width 0.635) (layer B.Cu) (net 15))
 (segment (start 66.675 56.495) (end 67.965 57.785) (width 0.635) (layer B.Cu) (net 15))
 (segment (start 66.675 54.61) (end 66.675 56.495) (width 0.635) (layer B.Cu) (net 15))
 (segment (start 67.965 57.785) (end 71.755 57.785) (width 0.635) (layer B.Cu) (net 15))
 (segment (start 78.105 54.61) (end 78.105 55.88) (width 0.635) (layer B.Cu) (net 4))
 (segment (start 78.105 55.88) (end 80.645 58.42) (width 0.635) (layer B.Cu) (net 4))
 (segment (start 90.805 58.42) (end 93.345 60.96) (width 0.635) (layer B.Cu) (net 4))
 (segment (start 80.645 58.42) (end 90.805 58.42) (width 0.635) (layer B.Cu) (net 4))
 (segment (start 93.345 64.77) (end 95.885 62.23) (width 0.635) (layer B.Cu) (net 16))
 (segment (start 95.885 62.23) (end 95.885 59.055) (width 0.635) (layer B.Cu) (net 16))
 (segment (start 93.345 56.515) (end 93.345 54.61) (width 0.635) (layer B.Cu) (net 16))
 (segment (start 95.885 59.055) (end 93.345 56.515) (width 0.635) (layer B.Cu) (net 16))
 (segment (start 93.345 68.58) (end 99.06 62.865) (width 0.635) (layer B.Cu) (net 14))
 (segment (start 99.06 62.865) (end 105.41 62.865) (width 0.635) (layer B.Cu) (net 14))
 (segment (start 93.345 72.39) (end 99.06 78.105) (width 0.635) (layer B.Cu) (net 8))
 (segment (start 99.06 78.105) (end 105.41 78.105) (width 0.635) (layer B.Cu) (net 8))
 (segment (start 93.345 86.36) (end 93.345 84.455) (width 0.635) (layer B.Cu) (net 11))
 (segment (start 93.345 84.455) (end 95.885 81.915) (width 0.635) (layer B.Cu) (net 11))
 (segment (start 95.885 78.74) (end 93.345 76.2) (width 0.635) (layer B.Cu) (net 11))
 (segment (start 95.885 81.915) (end 95.885 78.74) (width 0.635) (layer B.Cu) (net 11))
 (segment (start 78.105 86.36) (end 78.105 85.725) (width 0.635) (layer B.Cu) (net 12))
 (segment (start 78.105 85.725) (end 80.01 83.82) (width 0.635) (layer B.Cu) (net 12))
 (segment (start 89.535 83.82) (end 93.345 80.01) (width 0.635) (layer B.Cu) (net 12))
 (segment (start 80.01 83.82) (end 89.535 83.82) (width 0.635) (layer B.Cu) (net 12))
 (segment (start 64.675 56.495) (end 62.75 58.42) (width 0.635) (layer B.Cu) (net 19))
 (segment (start 64.675 54.61) (end 64.675 56.495) (width 0.635) (layer B.Cu) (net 19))
 (segment (start 55.88 58.42) (end 53.34 60.96) (width 0.635) (layer B.Cu) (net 19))
 (segment (start 62.75 58.42) (end 55.88 58.42) (width 0.635) (layer B.Cu) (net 19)))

